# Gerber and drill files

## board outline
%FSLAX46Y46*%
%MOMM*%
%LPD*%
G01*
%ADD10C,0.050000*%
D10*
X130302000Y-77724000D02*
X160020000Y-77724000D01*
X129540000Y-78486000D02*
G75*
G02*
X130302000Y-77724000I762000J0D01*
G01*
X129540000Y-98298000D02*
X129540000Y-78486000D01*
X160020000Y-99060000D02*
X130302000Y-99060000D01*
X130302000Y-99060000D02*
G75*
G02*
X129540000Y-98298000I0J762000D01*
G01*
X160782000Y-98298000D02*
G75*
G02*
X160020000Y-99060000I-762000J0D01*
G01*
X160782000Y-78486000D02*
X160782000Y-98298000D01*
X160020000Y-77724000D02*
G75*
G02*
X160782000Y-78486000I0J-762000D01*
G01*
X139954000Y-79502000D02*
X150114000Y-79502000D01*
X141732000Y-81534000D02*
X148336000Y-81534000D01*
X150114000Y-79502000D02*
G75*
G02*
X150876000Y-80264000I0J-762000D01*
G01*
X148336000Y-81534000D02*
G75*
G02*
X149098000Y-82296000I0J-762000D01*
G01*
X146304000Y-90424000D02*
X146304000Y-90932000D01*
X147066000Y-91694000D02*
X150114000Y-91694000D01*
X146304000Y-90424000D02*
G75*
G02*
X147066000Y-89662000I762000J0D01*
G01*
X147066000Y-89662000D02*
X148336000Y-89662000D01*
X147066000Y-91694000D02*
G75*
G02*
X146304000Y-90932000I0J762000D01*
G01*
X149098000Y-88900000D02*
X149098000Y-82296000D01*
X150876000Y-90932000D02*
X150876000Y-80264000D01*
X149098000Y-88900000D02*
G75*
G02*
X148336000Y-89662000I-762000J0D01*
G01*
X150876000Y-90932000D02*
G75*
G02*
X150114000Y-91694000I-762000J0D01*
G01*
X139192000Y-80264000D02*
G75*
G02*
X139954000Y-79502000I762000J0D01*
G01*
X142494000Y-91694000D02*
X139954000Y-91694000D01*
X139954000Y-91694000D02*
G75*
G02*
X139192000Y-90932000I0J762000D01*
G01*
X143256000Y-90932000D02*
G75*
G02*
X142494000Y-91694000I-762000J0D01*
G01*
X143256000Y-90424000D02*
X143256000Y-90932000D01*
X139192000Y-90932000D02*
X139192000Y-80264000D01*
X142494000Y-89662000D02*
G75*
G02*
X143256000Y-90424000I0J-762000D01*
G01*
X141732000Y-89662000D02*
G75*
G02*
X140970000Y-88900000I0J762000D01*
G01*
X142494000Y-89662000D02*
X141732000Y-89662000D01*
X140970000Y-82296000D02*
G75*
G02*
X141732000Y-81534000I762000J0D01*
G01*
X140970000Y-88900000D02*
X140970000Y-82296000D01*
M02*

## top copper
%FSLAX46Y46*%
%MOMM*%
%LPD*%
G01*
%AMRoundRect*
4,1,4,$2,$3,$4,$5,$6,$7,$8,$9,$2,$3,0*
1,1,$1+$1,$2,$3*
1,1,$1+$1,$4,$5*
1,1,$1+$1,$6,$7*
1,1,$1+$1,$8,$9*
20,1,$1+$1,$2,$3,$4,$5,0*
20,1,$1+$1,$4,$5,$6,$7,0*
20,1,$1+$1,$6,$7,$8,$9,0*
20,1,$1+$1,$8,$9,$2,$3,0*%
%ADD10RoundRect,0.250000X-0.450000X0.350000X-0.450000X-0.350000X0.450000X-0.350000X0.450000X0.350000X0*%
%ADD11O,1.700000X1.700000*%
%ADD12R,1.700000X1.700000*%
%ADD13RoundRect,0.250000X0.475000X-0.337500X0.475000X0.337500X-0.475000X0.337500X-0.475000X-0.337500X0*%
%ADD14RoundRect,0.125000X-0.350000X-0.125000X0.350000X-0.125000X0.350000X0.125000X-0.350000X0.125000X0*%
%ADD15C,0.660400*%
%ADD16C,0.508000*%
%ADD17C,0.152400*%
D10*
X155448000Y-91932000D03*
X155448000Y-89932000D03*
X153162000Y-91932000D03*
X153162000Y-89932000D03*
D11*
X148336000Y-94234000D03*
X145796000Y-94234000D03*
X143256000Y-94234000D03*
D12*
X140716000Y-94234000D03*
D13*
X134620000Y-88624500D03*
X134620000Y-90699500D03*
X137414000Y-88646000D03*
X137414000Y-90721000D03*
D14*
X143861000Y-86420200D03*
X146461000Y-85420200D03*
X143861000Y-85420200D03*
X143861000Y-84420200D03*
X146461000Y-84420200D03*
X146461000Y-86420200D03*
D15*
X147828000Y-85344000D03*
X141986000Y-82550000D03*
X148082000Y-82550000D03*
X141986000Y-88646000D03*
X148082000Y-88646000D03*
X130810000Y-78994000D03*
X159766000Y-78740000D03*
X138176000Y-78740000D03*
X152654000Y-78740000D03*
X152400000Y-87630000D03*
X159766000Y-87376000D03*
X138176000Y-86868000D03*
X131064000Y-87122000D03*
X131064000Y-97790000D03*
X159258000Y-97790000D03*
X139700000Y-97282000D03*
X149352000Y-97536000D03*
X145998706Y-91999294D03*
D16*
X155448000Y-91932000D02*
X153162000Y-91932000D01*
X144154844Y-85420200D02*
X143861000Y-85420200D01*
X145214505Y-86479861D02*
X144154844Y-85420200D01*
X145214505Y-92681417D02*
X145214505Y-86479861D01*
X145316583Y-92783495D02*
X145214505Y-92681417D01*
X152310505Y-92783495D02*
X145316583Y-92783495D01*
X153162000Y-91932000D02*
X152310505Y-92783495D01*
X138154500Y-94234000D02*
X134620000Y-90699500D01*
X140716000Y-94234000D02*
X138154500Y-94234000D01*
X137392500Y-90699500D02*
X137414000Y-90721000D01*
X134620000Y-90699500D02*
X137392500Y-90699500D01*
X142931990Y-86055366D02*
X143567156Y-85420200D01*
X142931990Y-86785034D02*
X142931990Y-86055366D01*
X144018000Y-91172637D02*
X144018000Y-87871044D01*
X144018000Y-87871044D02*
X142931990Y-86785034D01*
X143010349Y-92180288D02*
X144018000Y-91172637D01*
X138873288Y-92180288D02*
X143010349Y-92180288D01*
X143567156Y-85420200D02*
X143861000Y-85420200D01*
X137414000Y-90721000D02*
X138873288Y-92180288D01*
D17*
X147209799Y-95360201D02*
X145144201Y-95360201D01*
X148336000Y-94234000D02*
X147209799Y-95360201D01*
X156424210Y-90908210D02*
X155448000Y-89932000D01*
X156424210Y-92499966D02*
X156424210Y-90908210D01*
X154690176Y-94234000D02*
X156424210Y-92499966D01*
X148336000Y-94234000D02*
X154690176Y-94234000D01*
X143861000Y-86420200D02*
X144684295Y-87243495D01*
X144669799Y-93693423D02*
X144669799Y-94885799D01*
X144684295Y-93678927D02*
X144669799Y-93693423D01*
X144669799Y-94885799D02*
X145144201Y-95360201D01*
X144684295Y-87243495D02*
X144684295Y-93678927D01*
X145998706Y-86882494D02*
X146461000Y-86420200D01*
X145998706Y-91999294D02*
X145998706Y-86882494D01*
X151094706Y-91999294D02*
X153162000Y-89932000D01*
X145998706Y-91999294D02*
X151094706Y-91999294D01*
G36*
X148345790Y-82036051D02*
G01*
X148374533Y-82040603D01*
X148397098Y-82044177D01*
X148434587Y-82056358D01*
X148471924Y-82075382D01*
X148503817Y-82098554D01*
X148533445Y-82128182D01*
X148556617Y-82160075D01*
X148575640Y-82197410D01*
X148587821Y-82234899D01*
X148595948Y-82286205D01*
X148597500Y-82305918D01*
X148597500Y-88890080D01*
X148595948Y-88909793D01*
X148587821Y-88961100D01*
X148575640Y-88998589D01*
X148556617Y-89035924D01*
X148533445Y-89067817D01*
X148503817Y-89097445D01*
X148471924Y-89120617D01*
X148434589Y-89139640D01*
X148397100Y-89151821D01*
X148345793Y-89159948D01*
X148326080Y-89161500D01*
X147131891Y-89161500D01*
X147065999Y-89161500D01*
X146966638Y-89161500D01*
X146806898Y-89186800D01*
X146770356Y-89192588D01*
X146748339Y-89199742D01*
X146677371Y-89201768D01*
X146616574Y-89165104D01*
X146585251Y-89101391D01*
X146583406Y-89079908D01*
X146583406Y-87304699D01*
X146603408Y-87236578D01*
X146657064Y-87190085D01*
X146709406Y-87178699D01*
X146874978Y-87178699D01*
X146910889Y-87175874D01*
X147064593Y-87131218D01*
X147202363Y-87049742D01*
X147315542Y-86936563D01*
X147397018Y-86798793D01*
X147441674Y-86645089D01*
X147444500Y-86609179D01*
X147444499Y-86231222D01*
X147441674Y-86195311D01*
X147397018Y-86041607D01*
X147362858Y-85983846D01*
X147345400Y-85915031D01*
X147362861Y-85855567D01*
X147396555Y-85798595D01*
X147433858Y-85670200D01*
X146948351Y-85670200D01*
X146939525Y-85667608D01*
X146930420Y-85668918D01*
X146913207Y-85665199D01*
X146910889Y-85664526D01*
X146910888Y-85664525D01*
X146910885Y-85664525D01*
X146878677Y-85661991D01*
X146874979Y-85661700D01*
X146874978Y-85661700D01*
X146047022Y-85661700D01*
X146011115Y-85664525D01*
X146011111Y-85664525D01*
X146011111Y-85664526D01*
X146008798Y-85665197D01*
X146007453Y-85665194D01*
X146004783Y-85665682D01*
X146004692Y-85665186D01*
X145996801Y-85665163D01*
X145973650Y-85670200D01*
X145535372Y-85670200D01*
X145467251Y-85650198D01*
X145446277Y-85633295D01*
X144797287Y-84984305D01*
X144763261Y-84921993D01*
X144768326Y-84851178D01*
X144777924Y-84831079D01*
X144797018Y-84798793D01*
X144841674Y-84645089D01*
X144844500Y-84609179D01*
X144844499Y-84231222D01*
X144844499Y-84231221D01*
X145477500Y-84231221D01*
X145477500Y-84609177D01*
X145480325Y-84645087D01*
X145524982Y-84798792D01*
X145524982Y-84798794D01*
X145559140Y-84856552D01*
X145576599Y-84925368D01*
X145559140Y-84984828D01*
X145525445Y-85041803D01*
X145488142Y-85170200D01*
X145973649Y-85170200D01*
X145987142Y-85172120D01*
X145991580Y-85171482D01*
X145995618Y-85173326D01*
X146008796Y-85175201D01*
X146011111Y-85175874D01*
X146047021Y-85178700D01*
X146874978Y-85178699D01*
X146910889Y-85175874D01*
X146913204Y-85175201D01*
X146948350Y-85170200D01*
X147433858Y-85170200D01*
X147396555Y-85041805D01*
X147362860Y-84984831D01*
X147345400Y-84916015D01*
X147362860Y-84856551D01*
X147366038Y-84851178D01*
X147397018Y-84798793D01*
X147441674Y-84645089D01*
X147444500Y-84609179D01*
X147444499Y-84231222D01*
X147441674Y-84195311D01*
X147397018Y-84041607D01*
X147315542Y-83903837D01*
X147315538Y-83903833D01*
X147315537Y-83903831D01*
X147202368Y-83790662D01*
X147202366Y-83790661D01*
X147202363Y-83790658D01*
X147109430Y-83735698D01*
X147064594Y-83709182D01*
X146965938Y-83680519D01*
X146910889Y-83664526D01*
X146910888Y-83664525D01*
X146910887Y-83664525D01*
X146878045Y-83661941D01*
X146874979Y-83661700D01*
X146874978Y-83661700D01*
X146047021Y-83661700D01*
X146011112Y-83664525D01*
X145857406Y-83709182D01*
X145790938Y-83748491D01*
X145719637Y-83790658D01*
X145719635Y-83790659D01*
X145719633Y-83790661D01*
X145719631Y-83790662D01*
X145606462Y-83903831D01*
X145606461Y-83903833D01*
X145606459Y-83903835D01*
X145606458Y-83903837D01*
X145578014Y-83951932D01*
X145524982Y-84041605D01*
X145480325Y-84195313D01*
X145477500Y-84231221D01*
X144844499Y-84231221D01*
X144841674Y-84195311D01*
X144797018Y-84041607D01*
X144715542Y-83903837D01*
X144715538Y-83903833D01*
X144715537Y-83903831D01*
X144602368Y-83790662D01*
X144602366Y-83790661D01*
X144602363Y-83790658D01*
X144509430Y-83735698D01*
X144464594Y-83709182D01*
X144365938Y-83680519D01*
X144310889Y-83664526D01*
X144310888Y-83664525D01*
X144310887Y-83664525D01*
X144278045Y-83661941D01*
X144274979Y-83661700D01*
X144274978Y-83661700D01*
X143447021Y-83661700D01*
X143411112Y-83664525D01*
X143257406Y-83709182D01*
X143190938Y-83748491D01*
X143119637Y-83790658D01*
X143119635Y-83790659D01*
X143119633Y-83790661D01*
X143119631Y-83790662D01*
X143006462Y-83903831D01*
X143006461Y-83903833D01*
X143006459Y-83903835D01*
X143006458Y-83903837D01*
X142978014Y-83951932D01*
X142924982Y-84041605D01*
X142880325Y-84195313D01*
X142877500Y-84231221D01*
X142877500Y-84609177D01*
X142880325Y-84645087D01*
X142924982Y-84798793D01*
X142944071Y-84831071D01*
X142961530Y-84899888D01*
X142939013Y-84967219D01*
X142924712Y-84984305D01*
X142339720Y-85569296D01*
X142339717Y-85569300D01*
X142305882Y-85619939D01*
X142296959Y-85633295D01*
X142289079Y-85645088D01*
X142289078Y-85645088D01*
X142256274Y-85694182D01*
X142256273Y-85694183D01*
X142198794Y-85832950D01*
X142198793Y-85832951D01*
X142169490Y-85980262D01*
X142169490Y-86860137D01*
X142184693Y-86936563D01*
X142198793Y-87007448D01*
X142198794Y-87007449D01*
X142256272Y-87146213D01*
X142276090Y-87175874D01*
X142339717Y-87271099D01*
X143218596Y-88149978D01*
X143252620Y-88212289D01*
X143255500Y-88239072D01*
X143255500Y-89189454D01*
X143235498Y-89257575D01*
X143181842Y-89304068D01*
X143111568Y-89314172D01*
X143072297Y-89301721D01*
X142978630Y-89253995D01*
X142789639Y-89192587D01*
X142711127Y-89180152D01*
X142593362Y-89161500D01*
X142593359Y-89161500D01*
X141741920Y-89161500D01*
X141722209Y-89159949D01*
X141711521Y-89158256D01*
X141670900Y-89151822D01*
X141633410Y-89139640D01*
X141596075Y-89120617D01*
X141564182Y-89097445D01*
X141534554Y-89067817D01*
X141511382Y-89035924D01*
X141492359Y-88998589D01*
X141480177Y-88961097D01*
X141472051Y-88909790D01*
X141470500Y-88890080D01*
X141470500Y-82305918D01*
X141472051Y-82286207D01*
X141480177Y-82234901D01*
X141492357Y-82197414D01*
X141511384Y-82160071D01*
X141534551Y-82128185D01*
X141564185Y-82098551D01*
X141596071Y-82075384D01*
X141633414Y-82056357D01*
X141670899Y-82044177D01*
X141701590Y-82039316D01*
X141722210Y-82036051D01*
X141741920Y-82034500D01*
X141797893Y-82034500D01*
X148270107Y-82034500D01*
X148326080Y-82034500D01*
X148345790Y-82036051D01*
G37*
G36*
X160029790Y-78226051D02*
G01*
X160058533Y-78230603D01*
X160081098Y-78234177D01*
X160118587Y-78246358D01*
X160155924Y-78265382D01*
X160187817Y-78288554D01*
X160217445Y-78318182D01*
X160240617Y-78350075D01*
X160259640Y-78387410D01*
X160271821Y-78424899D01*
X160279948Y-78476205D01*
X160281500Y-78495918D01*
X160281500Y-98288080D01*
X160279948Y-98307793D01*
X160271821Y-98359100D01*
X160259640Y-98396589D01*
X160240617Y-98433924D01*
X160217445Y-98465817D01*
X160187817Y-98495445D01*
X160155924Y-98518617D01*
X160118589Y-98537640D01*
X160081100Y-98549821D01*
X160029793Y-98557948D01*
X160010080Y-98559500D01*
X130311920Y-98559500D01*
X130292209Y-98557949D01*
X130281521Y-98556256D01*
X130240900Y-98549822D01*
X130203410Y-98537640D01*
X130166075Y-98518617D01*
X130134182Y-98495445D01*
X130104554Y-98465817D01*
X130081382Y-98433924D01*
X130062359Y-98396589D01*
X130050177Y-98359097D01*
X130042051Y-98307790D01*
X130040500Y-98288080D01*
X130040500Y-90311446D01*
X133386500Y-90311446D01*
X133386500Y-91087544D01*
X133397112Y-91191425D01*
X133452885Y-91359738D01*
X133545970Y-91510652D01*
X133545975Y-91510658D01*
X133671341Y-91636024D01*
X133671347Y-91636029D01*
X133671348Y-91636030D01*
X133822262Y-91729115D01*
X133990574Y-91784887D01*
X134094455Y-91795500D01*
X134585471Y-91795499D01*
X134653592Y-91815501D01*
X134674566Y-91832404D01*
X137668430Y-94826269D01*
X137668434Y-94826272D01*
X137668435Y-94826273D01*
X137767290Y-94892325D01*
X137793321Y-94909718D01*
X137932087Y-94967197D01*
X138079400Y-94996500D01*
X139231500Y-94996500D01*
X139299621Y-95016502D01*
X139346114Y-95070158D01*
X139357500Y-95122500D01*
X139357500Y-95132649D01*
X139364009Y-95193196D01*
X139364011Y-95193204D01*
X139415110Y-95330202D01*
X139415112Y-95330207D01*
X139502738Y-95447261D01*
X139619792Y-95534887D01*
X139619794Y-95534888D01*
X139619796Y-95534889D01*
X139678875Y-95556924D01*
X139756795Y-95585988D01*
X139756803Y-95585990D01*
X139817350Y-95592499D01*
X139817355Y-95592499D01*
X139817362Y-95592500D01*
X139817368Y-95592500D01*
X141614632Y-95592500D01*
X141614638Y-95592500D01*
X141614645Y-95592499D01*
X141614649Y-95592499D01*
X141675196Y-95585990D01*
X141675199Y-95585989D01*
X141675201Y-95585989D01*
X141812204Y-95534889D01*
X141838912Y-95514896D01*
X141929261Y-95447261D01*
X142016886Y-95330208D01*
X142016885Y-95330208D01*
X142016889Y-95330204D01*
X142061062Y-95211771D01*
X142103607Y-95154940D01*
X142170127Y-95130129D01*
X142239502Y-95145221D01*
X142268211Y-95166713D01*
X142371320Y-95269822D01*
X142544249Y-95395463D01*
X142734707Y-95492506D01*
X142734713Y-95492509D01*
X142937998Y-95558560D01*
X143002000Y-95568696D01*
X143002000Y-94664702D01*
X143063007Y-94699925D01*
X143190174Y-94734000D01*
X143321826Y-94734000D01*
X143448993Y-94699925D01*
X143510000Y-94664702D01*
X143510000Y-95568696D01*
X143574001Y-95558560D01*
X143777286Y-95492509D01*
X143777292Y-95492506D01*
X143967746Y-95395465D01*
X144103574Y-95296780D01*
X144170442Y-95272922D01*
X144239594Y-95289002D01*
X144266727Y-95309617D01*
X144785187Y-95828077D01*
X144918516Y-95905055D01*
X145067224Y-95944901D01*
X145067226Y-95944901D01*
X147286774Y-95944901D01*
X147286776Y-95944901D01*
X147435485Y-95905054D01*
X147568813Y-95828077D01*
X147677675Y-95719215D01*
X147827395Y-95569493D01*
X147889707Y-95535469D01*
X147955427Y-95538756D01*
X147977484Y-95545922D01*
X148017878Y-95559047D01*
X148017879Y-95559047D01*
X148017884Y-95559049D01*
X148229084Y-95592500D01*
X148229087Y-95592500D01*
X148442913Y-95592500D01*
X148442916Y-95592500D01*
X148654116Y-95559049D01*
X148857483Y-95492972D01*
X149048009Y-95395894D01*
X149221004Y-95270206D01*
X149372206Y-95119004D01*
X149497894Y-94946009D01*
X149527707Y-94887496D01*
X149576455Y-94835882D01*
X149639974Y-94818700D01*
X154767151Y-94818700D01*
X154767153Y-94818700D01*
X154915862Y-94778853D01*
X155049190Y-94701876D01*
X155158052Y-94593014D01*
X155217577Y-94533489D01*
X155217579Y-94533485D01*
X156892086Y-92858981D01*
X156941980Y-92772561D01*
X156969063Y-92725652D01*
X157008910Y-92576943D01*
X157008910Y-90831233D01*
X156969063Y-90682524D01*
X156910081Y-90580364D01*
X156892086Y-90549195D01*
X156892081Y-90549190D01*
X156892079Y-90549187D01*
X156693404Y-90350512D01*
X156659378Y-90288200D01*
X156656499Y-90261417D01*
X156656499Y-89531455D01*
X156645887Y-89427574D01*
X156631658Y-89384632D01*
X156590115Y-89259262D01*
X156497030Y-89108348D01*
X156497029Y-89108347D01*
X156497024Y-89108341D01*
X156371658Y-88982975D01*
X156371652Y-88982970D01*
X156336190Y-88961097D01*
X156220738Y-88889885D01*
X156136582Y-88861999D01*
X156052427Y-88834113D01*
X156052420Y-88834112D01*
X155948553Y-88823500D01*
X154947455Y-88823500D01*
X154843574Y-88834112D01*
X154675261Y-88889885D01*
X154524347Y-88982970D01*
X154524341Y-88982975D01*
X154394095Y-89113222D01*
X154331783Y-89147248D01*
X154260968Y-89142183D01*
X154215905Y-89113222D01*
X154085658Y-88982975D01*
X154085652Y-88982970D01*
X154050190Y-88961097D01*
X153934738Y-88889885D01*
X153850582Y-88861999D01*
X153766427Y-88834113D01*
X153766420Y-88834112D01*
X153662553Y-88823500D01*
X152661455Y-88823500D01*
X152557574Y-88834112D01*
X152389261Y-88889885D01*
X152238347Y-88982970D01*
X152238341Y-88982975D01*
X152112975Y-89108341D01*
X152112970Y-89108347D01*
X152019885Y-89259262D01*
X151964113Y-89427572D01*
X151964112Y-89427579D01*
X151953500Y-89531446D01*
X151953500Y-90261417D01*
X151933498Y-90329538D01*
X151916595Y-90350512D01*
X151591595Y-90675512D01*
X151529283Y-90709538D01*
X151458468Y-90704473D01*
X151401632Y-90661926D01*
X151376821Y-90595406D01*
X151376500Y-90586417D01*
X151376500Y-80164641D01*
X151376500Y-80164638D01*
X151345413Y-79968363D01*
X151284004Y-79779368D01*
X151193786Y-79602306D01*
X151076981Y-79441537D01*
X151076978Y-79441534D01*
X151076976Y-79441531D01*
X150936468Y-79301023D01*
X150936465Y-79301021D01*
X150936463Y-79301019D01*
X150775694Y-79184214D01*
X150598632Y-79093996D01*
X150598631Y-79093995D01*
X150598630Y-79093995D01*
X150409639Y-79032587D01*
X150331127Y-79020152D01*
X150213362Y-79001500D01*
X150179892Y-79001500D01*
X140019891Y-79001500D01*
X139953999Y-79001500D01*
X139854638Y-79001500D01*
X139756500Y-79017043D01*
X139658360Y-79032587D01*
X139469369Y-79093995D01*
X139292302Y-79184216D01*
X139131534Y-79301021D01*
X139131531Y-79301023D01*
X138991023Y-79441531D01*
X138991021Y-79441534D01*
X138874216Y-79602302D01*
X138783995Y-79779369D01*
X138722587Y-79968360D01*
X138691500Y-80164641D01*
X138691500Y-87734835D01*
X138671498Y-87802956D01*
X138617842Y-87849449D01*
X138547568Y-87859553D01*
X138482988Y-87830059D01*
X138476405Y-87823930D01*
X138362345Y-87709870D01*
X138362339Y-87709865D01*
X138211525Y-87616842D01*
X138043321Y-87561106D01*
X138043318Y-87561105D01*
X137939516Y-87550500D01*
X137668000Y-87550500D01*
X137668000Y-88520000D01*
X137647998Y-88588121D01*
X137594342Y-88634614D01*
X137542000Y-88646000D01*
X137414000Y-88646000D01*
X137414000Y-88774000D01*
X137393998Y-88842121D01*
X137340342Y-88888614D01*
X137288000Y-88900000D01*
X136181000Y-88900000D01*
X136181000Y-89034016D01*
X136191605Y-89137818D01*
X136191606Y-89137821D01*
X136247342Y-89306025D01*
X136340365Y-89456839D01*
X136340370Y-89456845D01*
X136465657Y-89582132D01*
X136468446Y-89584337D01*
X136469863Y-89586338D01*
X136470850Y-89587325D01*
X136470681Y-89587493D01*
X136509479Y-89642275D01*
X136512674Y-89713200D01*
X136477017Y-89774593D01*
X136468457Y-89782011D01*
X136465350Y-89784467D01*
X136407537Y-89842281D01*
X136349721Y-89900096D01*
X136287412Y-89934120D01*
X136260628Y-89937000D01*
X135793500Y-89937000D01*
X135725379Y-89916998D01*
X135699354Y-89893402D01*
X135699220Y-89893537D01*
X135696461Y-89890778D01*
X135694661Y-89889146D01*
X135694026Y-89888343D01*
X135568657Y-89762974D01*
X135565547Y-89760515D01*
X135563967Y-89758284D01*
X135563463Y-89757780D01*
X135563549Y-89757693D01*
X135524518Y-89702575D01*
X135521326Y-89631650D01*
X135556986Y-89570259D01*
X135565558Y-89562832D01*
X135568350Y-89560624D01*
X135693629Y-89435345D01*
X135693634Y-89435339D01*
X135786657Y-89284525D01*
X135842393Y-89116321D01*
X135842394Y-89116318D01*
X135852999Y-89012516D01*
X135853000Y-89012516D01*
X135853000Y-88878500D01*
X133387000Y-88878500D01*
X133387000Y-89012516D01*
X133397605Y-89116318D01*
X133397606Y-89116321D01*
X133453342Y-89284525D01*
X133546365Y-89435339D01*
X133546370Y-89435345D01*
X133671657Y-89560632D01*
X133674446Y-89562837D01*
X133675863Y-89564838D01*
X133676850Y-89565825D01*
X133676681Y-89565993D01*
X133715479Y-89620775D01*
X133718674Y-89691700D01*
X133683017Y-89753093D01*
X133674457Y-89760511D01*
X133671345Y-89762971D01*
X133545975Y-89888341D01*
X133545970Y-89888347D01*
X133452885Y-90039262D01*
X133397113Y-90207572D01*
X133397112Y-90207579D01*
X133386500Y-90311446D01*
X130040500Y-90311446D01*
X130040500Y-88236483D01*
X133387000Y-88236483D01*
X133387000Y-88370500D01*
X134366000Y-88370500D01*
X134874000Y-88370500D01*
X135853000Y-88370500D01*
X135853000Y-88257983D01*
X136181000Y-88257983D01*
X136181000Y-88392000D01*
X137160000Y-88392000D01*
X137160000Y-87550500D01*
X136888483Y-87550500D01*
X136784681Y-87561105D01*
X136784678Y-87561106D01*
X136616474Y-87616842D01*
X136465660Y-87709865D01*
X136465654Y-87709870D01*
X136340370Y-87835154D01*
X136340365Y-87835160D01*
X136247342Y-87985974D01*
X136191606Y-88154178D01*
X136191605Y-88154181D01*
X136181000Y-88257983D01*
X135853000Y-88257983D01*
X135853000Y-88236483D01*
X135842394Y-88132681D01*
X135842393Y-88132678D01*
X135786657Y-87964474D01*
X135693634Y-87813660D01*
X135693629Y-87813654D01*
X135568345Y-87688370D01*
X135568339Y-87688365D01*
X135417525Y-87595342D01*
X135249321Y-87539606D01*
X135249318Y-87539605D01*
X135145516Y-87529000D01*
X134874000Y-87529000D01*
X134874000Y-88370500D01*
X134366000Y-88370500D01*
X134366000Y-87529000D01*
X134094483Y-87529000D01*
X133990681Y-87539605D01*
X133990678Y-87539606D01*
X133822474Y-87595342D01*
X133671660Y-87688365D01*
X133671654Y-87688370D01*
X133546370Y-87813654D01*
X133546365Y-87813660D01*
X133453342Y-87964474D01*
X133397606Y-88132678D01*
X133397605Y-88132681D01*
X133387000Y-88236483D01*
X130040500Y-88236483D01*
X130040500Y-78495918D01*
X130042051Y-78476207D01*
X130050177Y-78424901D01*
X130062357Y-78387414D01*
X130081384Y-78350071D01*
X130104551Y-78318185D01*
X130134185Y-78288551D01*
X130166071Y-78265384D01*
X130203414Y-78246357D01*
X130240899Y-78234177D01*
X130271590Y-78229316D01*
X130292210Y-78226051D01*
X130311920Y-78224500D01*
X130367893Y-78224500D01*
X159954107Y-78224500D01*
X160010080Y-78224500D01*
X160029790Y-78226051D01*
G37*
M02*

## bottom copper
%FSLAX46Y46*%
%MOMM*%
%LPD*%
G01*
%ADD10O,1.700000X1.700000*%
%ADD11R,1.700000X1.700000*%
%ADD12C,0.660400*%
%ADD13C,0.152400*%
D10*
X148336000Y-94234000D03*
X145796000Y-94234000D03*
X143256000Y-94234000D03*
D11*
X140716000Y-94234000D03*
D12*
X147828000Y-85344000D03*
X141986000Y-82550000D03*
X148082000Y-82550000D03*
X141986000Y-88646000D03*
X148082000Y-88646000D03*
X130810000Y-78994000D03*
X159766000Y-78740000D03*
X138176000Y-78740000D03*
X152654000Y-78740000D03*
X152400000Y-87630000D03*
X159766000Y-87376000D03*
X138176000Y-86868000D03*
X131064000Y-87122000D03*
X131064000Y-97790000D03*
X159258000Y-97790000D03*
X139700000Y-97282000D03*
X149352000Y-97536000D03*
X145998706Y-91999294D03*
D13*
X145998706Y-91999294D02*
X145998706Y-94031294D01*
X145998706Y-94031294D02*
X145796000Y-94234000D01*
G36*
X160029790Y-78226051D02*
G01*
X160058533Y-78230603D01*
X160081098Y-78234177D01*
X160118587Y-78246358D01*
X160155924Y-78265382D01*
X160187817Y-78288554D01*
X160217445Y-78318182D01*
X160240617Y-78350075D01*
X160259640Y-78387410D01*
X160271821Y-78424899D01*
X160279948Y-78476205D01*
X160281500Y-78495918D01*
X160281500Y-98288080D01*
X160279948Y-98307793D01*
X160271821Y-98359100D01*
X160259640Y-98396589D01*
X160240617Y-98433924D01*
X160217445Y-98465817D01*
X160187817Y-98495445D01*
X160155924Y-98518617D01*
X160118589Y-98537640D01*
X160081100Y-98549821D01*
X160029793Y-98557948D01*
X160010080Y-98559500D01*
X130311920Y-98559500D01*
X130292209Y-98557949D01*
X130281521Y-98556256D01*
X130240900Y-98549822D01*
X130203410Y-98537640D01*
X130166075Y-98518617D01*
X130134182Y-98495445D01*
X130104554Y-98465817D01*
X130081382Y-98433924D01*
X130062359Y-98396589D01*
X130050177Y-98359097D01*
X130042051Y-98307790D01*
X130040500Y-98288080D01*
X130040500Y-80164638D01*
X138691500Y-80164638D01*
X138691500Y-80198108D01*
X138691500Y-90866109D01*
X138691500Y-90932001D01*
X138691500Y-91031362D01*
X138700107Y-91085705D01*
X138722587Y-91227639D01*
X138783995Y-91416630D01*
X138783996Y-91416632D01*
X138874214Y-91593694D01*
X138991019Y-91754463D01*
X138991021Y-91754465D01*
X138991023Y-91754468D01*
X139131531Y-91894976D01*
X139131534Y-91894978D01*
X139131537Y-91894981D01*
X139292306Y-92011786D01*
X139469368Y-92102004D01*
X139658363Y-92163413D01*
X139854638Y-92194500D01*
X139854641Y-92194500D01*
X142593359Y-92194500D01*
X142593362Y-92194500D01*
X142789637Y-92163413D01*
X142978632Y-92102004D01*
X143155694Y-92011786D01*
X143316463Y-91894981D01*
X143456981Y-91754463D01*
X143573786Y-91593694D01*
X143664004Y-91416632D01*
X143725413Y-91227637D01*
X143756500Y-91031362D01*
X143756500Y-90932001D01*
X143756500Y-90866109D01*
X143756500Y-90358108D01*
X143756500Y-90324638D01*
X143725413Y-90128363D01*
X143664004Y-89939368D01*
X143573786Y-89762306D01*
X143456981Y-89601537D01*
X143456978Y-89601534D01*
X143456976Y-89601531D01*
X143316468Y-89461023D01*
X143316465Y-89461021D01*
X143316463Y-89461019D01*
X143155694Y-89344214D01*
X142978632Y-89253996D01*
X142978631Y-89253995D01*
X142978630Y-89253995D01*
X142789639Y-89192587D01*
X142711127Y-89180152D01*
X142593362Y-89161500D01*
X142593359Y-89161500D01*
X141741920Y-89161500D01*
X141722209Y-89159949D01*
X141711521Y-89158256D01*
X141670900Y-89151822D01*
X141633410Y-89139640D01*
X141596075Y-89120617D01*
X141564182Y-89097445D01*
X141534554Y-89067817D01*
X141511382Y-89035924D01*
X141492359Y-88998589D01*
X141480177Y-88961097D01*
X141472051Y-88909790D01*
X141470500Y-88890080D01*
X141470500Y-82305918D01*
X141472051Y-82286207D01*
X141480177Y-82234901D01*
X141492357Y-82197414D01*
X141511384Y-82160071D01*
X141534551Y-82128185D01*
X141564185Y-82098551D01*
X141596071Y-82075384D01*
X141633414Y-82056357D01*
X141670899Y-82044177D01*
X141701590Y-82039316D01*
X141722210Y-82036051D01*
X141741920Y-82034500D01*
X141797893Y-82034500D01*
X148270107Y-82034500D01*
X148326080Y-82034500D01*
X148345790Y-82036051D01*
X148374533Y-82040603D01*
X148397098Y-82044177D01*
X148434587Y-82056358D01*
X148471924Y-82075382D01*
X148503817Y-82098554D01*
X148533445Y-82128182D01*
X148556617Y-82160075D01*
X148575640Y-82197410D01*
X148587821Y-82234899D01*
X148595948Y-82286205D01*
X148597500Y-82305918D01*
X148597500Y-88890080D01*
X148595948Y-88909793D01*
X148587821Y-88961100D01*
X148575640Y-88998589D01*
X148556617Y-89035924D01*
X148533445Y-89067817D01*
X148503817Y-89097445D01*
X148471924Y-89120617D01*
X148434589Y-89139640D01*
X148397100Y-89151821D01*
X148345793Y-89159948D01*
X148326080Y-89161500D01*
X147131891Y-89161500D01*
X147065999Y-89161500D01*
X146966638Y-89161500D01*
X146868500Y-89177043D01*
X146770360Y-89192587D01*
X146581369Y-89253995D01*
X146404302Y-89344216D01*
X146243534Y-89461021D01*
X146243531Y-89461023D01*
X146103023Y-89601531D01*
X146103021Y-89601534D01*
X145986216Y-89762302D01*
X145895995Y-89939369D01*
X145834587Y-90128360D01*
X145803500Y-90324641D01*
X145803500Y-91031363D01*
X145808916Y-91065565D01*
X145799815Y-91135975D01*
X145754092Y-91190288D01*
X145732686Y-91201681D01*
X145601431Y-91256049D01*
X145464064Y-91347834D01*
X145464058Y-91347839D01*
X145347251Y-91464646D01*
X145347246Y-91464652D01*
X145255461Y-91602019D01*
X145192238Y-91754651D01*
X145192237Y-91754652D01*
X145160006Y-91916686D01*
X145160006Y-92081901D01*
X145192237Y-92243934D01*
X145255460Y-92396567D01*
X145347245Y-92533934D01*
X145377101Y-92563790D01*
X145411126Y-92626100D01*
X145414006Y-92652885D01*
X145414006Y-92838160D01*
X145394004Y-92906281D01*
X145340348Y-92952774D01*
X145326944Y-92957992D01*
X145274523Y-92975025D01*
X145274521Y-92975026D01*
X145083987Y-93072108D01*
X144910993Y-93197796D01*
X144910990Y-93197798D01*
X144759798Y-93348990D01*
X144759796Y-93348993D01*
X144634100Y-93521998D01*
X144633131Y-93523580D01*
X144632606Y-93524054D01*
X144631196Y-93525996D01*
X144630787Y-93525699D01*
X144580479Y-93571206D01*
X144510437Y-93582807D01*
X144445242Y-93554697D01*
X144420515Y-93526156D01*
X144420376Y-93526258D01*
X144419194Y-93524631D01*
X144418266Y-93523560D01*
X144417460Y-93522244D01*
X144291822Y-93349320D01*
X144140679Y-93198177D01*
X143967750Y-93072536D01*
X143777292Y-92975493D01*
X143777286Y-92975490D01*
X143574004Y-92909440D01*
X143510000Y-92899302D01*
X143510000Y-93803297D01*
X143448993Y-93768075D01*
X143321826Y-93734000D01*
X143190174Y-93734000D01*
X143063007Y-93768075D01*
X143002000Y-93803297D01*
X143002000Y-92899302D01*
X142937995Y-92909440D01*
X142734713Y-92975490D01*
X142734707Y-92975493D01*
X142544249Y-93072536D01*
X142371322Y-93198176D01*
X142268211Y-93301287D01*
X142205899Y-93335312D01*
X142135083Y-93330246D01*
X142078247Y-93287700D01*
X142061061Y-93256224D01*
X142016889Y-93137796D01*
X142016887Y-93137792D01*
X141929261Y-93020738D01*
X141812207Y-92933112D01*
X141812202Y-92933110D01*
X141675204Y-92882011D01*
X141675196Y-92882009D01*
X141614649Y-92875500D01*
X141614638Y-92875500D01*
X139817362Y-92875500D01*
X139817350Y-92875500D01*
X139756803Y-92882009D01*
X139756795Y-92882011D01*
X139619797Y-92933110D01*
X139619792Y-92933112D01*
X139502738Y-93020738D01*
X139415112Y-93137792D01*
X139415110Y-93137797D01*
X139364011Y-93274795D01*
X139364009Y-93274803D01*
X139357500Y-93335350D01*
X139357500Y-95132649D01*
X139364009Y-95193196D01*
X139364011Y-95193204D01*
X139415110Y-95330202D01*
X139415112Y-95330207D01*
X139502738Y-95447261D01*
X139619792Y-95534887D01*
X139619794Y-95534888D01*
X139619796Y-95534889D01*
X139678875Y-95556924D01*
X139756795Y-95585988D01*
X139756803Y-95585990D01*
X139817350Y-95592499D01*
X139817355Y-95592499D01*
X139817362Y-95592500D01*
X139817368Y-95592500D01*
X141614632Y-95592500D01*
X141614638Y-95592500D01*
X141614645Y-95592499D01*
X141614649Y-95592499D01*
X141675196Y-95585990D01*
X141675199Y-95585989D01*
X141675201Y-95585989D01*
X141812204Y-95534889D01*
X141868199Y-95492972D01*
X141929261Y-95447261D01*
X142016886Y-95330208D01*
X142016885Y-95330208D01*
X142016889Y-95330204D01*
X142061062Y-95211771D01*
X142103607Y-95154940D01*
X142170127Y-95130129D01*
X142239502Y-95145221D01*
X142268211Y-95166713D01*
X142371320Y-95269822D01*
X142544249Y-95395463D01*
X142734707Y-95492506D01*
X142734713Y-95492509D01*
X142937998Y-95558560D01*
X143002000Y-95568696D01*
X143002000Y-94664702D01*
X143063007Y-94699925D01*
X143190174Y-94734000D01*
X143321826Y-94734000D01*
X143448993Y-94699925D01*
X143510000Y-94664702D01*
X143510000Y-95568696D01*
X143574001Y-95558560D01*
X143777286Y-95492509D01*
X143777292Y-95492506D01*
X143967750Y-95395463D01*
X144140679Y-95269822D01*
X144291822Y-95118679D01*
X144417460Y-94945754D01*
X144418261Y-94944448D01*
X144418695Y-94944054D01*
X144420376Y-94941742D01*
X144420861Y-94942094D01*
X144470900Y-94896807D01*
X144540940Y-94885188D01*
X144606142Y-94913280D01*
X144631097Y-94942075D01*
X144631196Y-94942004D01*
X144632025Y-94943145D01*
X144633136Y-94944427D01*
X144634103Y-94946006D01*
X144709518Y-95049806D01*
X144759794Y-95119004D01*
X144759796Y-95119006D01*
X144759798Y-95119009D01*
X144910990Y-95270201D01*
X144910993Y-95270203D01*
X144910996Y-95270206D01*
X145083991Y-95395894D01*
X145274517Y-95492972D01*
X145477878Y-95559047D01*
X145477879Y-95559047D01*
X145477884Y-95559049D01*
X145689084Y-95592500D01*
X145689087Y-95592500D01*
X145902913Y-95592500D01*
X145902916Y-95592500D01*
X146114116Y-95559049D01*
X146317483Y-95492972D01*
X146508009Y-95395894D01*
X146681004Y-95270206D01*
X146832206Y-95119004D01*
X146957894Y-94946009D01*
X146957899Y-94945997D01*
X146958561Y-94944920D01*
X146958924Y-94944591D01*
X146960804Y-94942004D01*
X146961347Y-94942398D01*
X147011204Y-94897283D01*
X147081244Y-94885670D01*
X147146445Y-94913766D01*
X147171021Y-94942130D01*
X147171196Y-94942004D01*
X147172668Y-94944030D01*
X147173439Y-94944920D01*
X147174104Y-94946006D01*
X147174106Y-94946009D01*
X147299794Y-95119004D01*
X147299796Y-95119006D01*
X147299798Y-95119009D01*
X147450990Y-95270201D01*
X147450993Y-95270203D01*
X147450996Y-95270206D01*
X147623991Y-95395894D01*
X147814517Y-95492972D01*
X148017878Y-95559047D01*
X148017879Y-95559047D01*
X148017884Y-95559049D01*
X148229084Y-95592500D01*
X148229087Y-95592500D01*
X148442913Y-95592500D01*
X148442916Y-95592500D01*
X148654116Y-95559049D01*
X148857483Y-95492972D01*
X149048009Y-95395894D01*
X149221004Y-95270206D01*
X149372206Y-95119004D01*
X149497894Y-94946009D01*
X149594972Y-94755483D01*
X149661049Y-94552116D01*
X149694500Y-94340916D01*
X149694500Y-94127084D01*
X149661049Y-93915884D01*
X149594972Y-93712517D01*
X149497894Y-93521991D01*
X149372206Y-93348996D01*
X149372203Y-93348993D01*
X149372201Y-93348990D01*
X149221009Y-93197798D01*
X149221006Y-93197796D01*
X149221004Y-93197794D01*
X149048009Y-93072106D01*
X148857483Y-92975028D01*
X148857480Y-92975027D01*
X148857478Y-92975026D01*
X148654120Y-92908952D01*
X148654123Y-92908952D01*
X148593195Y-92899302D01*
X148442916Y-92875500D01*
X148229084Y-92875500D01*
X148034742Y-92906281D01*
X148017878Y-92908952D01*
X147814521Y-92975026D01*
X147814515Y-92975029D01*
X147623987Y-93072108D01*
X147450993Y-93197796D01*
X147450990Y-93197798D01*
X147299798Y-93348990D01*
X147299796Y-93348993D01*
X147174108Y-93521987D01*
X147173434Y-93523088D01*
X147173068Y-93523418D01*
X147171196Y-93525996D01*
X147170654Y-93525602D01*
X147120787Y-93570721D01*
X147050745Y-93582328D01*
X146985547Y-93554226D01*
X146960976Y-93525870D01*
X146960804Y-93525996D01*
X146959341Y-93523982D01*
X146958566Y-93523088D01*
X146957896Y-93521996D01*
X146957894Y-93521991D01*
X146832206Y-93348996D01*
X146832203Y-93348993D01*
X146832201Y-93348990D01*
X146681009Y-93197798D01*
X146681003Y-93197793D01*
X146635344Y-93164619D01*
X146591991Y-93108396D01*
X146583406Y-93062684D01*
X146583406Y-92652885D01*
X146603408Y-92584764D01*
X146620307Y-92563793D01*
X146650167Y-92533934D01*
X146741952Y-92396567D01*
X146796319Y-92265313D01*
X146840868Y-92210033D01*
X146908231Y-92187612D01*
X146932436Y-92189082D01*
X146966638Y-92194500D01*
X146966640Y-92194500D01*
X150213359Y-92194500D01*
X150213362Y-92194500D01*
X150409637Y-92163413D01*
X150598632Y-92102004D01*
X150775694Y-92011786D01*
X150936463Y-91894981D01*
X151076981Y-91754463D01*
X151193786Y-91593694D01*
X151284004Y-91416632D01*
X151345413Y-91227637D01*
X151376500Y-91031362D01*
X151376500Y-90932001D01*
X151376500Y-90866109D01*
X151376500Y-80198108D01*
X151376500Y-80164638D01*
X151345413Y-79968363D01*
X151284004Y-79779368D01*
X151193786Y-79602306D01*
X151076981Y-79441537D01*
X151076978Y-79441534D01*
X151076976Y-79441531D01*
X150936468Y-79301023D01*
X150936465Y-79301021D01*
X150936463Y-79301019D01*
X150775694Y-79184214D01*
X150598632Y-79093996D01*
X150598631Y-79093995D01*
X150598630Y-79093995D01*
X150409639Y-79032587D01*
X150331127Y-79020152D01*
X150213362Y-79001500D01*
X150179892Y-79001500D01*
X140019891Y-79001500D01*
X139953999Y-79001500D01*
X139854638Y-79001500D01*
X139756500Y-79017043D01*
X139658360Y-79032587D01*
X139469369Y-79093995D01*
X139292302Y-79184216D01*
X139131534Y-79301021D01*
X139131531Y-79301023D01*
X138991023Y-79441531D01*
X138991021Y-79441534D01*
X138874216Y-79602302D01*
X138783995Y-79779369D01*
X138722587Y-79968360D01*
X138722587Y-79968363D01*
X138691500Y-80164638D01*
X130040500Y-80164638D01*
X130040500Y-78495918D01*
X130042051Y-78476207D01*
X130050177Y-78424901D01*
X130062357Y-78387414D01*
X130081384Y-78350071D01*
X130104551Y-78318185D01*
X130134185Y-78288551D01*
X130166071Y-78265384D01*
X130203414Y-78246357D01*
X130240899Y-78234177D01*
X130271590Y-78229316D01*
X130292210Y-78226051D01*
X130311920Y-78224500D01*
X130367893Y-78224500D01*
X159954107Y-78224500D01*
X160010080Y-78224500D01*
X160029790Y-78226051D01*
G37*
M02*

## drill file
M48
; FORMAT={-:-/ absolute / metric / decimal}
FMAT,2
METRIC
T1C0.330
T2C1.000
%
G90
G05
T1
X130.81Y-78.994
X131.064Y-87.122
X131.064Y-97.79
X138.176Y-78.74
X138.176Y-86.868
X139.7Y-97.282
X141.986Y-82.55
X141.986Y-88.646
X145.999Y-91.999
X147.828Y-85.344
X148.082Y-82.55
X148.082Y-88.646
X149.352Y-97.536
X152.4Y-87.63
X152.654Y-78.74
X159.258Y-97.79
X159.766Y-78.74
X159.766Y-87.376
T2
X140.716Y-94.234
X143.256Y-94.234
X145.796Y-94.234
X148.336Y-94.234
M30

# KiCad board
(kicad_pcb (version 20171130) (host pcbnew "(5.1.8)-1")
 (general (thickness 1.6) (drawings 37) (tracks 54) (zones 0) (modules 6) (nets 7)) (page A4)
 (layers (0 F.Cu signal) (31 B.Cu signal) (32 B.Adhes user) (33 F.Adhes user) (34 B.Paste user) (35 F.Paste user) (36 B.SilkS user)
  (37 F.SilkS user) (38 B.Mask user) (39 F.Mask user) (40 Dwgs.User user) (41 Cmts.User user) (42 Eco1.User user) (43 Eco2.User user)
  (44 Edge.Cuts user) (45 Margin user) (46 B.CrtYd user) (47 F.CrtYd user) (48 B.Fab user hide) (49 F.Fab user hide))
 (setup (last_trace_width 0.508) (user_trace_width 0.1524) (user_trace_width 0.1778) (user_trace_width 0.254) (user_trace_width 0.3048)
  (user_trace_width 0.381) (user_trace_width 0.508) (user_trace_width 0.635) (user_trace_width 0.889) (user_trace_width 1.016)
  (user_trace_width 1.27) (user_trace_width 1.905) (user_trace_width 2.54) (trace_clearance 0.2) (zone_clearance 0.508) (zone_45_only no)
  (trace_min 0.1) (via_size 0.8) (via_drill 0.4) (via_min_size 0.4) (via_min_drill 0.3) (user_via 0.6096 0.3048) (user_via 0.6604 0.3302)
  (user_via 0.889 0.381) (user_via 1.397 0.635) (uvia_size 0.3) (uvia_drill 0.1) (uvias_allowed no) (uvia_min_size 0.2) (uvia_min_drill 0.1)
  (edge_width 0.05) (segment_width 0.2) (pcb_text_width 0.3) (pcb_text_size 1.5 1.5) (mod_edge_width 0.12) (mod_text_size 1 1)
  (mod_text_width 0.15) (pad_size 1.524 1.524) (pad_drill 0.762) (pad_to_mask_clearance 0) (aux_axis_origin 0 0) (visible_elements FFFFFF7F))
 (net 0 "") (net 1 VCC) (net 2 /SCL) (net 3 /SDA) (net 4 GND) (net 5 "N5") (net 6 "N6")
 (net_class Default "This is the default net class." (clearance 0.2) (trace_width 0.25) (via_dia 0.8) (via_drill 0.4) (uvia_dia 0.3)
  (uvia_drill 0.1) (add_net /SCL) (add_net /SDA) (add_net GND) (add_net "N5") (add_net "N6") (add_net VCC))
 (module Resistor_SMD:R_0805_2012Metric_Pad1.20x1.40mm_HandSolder (layer F.Cu) (at 155.448 90.932 270)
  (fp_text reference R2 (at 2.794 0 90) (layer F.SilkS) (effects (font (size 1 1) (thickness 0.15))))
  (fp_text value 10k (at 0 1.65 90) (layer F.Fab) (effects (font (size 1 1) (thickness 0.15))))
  (pad 2 smd roundrect (at 1 0 270) (size 1.2 1.4) (layers F.Cu F.Paste F.Mask) (roundrect_rratio 0.208333) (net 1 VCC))
  (pad 1 smd roundrect (at -1 0 270) (size 1.2 1.4) (layers F.Cu F.Paste F.Mask) (roundrect_rratio 0.208333) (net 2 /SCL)))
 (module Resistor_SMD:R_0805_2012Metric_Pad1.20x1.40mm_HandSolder (layer F.Cu) (at 153.162 90.932 270)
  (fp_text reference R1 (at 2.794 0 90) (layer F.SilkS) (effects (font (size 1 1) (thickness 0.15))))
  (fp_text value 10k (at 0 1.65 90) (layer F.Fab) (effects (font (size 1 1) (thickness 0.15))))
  (pad 2 smd roundrect (at 1 0 270) (size 1.2 1.4) (layers F.Cu F.Paste F.Mask) (roundrect_rratio 0.208333) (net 1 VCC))
  (pad 1 smd roundrect (at -1 0 270) (size 1.2 1.4) (layers F.Cu F.Paste F.Mask) (roundrect_rratio 0.208333) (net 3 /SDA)))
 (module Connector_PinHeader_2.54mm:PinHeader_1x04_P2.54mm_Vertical (layer F.Cu) (at 140.716 94.234 90)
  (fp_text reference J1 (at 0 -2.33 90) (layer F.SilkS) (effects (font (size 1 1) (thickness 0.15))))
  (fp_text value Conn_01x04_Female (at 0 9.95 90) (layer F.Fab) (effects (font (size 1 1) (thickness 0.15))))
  (pad 4 thru_hole oval (at 0 7.62 90) (size 1.7 1.7) (drill 1) (layers *.Cu *.Mask) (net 2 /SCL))
  (pad 3 thru_hole oval (at 0 5.08 90) (size 1.7 1.7) (drill 1) (layers *.Cu *.Mask) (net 3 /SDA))
  (pad 2 thru_hole oval (at 0 2.54 90) (size 1.7 1.7) (drill 1) (layers *.Cu *.Mask) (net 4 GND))
  (pad 1 thru_hole rect (at 0 0 90) (size 1.7 1.7) (drill 1) (layers *.Cu *.Mask) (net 1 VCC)))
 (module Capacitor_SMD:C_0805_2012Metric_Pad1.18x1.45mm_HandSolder (layer F.Cu) (at 134.62 89.662 90)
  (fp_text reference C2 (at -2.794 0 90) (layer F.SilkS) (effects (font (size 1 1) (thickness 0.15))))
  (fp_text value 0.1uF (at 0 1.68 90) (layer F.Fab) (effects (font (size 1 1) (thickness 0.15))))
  (pad 2 smd roundrect (at 1.0375 0 90) (size 1.175 1.45) (layers F.Cu F.Paste F.Mask) (roundrect_rratio 0.212766) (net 4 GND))
  (pad 1 smd roundrect (at -1.0375 0 90) (size 1.175 1.45) (layers F.Cu F.Paste F.Mask) (roundrect_rratio 0.212766) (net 1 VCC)))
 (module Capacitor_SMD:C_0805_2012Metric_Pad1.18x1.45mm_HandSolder (layer F.Cu) (at 137.414 89.6835 90)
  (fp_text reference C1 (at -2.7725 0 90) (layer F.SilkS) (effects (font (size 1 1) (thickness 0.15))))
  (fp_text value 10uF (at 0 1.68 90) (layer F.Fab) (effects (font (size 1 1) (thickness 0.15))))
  (pad 2 smd roundrect (at 1.0375 0 90) (size 1.175 1.45) (layers F.Cu F.Paste F.Mask) (roundrect_rratio 0.212766) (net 4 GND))
  (pad 1 smd roundrect (at -1.0375 0 90) (size 1.175 1.45) (layers F.Cu F.Paste F.Mask) (roundrect_rratio 0.212766) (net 1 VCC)))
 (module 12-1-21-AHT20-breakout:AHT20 (layer F.Cu) (at 145.542 84.582)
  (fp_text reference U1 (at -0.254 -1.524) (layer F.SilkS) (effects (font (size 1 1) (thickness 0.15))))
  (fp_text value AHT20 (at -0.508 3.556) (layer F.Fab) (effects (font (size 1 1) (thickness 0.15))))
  (pad 3 smd roundrect (at -1.681 1.8382) (size 0.95 0.5) (layers F.Cu F.Paste F.Mask) (roundrect_rratio 0.25) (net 2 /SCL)
   (solder_mask_margin 0.0508))
  (pad 5 smd roundrect (at 0.919 0.8382) (size 0.95 0.5) (layers F.Cu F.Paste F.Mask) (roundrect_rratio 0.25) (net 4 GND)
   (solder_mask_margin 0.0508))
  (pad 2 smd roundrect (at -1.681 0.8382) (size 0.95 0.5) (layers F.Cu F.Paste F.Mask) (roundrect_rratio 0.25) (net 1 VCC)
   (solder_mask_margin 0.0508))
  (pad 1 smd roundrect (at -1.681 -0.1618) (size 0.95 0.5) (layers F.Cu F.Paste F.Mask) (roundrect_rratio 0.25) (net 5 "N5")
   (solder_mask_margin 0.0508))
  (pad 6 smd roundrect (at 0.919 -0.1618) (size 0.95 0.5) (layers F.Cu F.Paste F.Mask) (roundrect_rratio 0.25) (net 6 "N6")
   (solder_mask_margin 0.0508))
  (pad 4 smd roundrect (at 0.919 1.8382) (size 0.95 0.5) (layers F.Cu F.Paste F.Mask) (roundrect_rratio 0.25) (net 3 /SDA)
   (solder_mask_margin 0.0508)))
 (gr_line (start 130.302 77.724) (end 160.02 77.724) (layer Edge.Cuts) (width 0.05))
 (gr_arc (start 130.302 78.486) (end 130.302 77.724) (angle -90) (layer Edge.Cuts) (width 0.05))
 (gr_line (start 129.54 98.298) (end 129.54 78.486) (layer Edge.Cuts) (width 0.05))
 (gr_line (start 160.02 99.06) (end 130.302 99.06) (layer Edge.Cuts) (width 0.05))
 (gr_arc (start 130.302 98.298) (end 129.54 98.298) (angle -90) (layer Edge.Cuts) (width 0.05))
 (gr_arc (start 160.02 98.298) (end 160.02 99.06) (angle -90) (layer Edge.Cuts) (width 0.05))
 (gr_line (start 160.782 78.486) (end 160.782 98.298) (layer Edge.Cuts) (width 0.05))
 (gr_arc (start 160.02 78.486) (end 160.782 78.486) (angle -90) (layer Edge.Cuts) (width 0.05))
 (gr_line (start 139.954 79.502) (end 150.114 79.502) (layer Edge.Cuts) (width 0.05))
 (gr_line (start 141.732 81.534) (end 148.336 81.534) (layer Edge.Cuts) (width 0.05))
 (gr_arc (start 150.114 80.264) (end 150.114 79.502) (angle 90) (layer Edge.Cuts) (width 0.05))
 (gr_arc (start 148.336 82.296) (end 148.336 81.534) (angle 90) (layer Edge.Cuts) (width 0.05))
 (gr_line (start 146.304 90.424) (end 146.304 90.932) (layer Edge.Cuts) (width 0.05))
 (gr_line (start 147.066 91.694) (end 150.114 91.694) (layer Edge.Cuts) (width 0.05))
 (gr_arc (start 147.066 90.424) (end 146.304 90.424) (angle 90) (layer Edge.Cuts) (width 0.05))
 (gr_line (start 147.066 89.662) (end 148.336 89.662) (layer Edge.Cuts) (width 0.05))
 (gr_arc (start 147.066 90.932) (end 147.066 91.694) (angle 90) (layer Edge.Cuts) (width 0.05))
 (gr_line (start 149.098 88.9) (end 149.098 82.296) (layer Edge.Cuts) (width 0.05))
 (gr_line (start 150.876 90.932) (end 150.876 80.264) (layer Edge.Cuts) (width 0.05))
 (gr_arc (start 148.336 88.9) (end 149.098 88.9) (angle 90) (layer Edge.Cuts) (width 0.05))
 (gr_arc (start 150.114 90.932) (end 150.876 90.932) (angle 90) (layer Edge.Cuts) (width 0.05))
 (gr_arc (start 139.954 80.264) (end 139.954 79.502) (angle -90) (layer Edge.Cuts) (width 0.05))
 (gr_line (start 142.494 91.694) (end 139.954 91.694) (layer Edge.Cuts) (width 0.05))
 (gr_arc (start 139.954 90.932) (end 139.192 90.932) (angle -90) (layer Edge.Cuts) (width 0.05))
 (gr_arc (start 142.494 90.932) (end 142.494 91.694) (angle -90) (layer Edge.Cuts) (width 0.05))
 (gr_line (start 143.256 90.424) (end 143.256 90.932) (layer Edge.Cuts) (width 0.05))
 (gr_line (start 139.192 90.932) (end 139.192 80.264) (layer Edge.Cuts) (width 0.05))
 (gr_arc (start 142.494 90.424) (end 143.256 90.424) (angle -90) (layer Edge.Cuts) (width 0.05))
 (gr_arc (start 141.732 88.9) (end 140.97 88.9) (angle -90) (layer Edge.Cuts) (width 0.05))
 (gr_line (start 142.494 89.662) (end 141.732 89.662) (layer Edge.Cuts) (width 0.05))
 (gr_arc (start 141.732 82.296) (end 141.732 81.534) (angle -90) (layer Edge.Cuts) (width 0.05))
 (gr_line (start 140.97 88.9) (end 140.97 82.296) (layer Edge.Cuts) (width 0.05))
 (via (at 147.828 85.344) (size 0.6604) (drill 0.3302) (layers F.Cu B.Cu) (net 4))
 (via (at 141.986 82.55) (size 0.6604) (drill 0.3302) (layers F.Cu B.Cu) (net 4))
 (via (at 148.082 82.55) (size 0.6604) (drill 0.3302) (layers F.Cu B.Cu) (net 4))
 (via (at 141.986 88.646) (size 0.6604) (drill 0.3302) (layers F.Cu B.Cu) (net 4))
 (via (at 148.082 88.646) (size 0.6604) (drill 0.3302) (layers F.Cu B.Cu) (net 4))
 (via (at 130.81 78.994) (size 0.6604) (drill 0.3302) (layers F.Cu B.Cu) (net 4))
 (via (at 159.766 78.74) (size 0.6604) (drill 0.3302) (layers F.Cu B.Cu) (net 4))
 (via (at 138.176 78.74) (size 0.6604) (drill 0.3302) (layers F.Cu B.Cu) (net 4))
 (via (at 152.654 78.74) (size 0.6604) (drill 0.3302) (layers F.Cu B.Cu) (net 4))
 (via (at 152.4 87.63) (size 0.6604) (drill 0.3302) (layers F.Cu B.Cu) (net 4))
 (via (at 159.766 87.376) (size 0.6604) (drill 0.3302) (layers F.Cu B.Cu) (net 4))
 (via (at 138.176 86.868) (size 0.6604) (drill 0.3302) (layers F.Cu B.Cu) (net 4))
 (via (at 131.064 87.122) (size 0.6604) (drill 0.3302) (layers F.Cu B.Cu) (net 4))
 (via (at 131.064 97.79) (size 0.6604) (drill 0.3302) (layers F.Cu B.Cu) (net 4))
 (via (at 159.258 97.79) (size 0.6604) (drill 0.3302) (layers F.Cu B.Cu) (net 4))
 (via (at 139.7 97.282) (size 0.6604) (drill 0.3302) (layers F.Cu B.Cu) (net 4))
 (via (at 149.352 97.536) (size 0.6604) (drill 0.3302) (layers F.Cu B.Cu) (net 4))
 (segment (start 155.448 91.932) (end 153.162 91.932) (width 0.508) (layer F.Cu) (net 1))
 (segment (start 144.154844 85.4202) (end 143.861 85.4202) (width 0.508) (layer F.Cu) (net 1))
 (segment (start 145.214505 86.479861) (end 144.154844 85.4202) (width 0.508) (layer F.Cu) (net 1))
 (segment (start 145.214505 92.681417) (end 145.214505 86.479861) (width 0.508) (layer F.Cu) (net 1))
 (segment (start 145.316583 92.783495) (end 145.214505 92.681417) (width 0.508) (layer F.Cu) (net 1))
 (segment (start 152.310505 92.783495) (end 145.316583 92.783495) (width 0.508) (layer F.Cu) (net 1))
 (segment (start 153.162 91.932) (end 152.310505 92.783495) (width 0.508) (layer F.Cu) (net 1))
 (segment (start 138.1545 94.234) (end 134.62 90.6995) (width 0.508) (layer F.Cu) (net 1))
 (segment (start 140.716 94.234) (end 138.1545 94.234) (width 0.508) (layer F.Cu) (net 1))
 (segment (start 137.3925 90.6995) (end 137.414 90.721) (width 0.508) (layer F.Cu) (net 1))
 (segment (start 134.62 90.6995) (end 137.3925 90.6995) (width 0.508) (layer F.Cu) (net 1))
 (segment (start 142.93199 86.055366) (end 143.567156 85.4202) (width 0.508) (layer F.Cu) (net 1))
 (segment (start 142.93199 86.785034) (end 142.93199 86.055366) (width 0.508) (layer F.Cu) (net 1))
 (segment (start 144.018 91.172637) (end 144.018 87.871044) (width 0.508) (layer F.Cu) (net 1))
 (segment (start 144.018 87.871044) (end 142.93199 86.785034) (width 0.508) (layer F.Cu) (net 1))
 (segment (start 143.010349 92.180288) (end 144.018 91.172637) (width 0.508) (layer F.Cu) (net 1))
 (segment (start 138.873288 92.180288) (end 143.010349 92.180288) (width 0.508) (layer F.Cu) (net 1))
 (segment (start 143.567156 85.4202) (end 143.861 85.4202) (width 0.508) (layer F.Cu) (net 1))
 (segment (start 137.414 90.721) (end 138.873288 92.180288) (width 0.508) (layer F.Cu) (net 1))
 (segment (start 147.209799 95.360201) (end 145.144201 95.360201) (width 0.1524) (layer F.Cu) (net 2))
 (segment (start 148.336 94.234) (end 147.209799 95.360201) (width 0.1524) (layer F.Cu) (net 2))
 (segment (start 156.42421 90.90821) (end 155.448 89.932) (width 0.1524) (layer F.Cu) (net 2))
 (segment (start 156.42421 92.499966) (end 156.42421 90.90821) (width 0.1524) (layer F.Cu) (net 2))
 (segment (start 154.690176 94.234) (end 156.42421 92.499966) (width 0.1524) (layer F.Cu) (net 2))
 (segment (start 148.336 94.234) (end 154.690176 94.234) (width 0.1524) (layer F.Cu) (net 2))
 (segment (start 143.861 86.4202) (end 144.684295 87.243495) (width 0.1524) (layer F.Cu) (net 2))
 (segment (start 144.669799 93.693423) (end 144.669799 94.885799) (width 0.1524) (layer F.Cu) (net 2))
 (segment (start 144.684295 93.678927) (end 144.669799 93.693423) (width 0.1524) (layer F.Cu) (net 2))
 (segment (start 144.669799 94.885799) (end 145.144201 95.360201) (width 0.1524) (layer F.Cu) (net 2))
 (segment (start 144.684295 87.243495) (end 144.684295 93.678927) (width 0.1524) (layer F.Cu) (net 2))
 (segment (start 145.998706 91.999294) (end 145.998706 94.031294) (width 0.1524) (layer B.Cu) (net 3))
 (segment (start 145.998706 94.031294) (end 145.796 94.234) (width 0.1524) (layer B.Cu) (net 3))
 (segment (start 145.998706 86.882494) (end 146.461 86.4202) (width 0.1524) (layer F.Cu) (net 3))
 (segment (start 145.998706 91.999294) (end 145.998706 86.882494) (width 0.1524) (layer F.Cu) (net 3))
 (via (at 145.998706 91.999294) (size 0.6604) (drill 0.3302) (layers F.Cu B.Cu) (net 3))
 (segment (start 151.094706 91.999294) (end 153.162 89.932) (width 0.1524) (layer F.Cu) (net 3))
 (segment (start 145.998706 91.999294) (end 151.094706 91.999294) (width 0.1524) (layer F.Cu) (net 3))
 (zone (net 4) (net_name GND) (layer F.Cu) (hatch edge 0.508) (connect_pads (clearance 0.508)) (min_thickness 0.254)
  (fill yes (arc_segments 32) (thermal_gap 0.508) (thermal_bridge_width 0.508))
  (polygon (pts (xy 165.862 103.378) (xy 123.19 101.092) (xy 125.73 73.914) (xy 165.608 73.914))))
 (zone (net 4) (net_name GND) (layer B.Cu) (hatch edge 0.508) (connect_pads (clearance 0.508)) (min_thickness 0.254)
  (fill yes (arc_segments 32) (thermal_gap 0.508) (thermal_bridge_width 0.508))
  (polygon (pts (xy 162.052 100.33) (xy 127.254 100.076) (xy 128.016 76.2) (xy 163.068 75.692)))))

